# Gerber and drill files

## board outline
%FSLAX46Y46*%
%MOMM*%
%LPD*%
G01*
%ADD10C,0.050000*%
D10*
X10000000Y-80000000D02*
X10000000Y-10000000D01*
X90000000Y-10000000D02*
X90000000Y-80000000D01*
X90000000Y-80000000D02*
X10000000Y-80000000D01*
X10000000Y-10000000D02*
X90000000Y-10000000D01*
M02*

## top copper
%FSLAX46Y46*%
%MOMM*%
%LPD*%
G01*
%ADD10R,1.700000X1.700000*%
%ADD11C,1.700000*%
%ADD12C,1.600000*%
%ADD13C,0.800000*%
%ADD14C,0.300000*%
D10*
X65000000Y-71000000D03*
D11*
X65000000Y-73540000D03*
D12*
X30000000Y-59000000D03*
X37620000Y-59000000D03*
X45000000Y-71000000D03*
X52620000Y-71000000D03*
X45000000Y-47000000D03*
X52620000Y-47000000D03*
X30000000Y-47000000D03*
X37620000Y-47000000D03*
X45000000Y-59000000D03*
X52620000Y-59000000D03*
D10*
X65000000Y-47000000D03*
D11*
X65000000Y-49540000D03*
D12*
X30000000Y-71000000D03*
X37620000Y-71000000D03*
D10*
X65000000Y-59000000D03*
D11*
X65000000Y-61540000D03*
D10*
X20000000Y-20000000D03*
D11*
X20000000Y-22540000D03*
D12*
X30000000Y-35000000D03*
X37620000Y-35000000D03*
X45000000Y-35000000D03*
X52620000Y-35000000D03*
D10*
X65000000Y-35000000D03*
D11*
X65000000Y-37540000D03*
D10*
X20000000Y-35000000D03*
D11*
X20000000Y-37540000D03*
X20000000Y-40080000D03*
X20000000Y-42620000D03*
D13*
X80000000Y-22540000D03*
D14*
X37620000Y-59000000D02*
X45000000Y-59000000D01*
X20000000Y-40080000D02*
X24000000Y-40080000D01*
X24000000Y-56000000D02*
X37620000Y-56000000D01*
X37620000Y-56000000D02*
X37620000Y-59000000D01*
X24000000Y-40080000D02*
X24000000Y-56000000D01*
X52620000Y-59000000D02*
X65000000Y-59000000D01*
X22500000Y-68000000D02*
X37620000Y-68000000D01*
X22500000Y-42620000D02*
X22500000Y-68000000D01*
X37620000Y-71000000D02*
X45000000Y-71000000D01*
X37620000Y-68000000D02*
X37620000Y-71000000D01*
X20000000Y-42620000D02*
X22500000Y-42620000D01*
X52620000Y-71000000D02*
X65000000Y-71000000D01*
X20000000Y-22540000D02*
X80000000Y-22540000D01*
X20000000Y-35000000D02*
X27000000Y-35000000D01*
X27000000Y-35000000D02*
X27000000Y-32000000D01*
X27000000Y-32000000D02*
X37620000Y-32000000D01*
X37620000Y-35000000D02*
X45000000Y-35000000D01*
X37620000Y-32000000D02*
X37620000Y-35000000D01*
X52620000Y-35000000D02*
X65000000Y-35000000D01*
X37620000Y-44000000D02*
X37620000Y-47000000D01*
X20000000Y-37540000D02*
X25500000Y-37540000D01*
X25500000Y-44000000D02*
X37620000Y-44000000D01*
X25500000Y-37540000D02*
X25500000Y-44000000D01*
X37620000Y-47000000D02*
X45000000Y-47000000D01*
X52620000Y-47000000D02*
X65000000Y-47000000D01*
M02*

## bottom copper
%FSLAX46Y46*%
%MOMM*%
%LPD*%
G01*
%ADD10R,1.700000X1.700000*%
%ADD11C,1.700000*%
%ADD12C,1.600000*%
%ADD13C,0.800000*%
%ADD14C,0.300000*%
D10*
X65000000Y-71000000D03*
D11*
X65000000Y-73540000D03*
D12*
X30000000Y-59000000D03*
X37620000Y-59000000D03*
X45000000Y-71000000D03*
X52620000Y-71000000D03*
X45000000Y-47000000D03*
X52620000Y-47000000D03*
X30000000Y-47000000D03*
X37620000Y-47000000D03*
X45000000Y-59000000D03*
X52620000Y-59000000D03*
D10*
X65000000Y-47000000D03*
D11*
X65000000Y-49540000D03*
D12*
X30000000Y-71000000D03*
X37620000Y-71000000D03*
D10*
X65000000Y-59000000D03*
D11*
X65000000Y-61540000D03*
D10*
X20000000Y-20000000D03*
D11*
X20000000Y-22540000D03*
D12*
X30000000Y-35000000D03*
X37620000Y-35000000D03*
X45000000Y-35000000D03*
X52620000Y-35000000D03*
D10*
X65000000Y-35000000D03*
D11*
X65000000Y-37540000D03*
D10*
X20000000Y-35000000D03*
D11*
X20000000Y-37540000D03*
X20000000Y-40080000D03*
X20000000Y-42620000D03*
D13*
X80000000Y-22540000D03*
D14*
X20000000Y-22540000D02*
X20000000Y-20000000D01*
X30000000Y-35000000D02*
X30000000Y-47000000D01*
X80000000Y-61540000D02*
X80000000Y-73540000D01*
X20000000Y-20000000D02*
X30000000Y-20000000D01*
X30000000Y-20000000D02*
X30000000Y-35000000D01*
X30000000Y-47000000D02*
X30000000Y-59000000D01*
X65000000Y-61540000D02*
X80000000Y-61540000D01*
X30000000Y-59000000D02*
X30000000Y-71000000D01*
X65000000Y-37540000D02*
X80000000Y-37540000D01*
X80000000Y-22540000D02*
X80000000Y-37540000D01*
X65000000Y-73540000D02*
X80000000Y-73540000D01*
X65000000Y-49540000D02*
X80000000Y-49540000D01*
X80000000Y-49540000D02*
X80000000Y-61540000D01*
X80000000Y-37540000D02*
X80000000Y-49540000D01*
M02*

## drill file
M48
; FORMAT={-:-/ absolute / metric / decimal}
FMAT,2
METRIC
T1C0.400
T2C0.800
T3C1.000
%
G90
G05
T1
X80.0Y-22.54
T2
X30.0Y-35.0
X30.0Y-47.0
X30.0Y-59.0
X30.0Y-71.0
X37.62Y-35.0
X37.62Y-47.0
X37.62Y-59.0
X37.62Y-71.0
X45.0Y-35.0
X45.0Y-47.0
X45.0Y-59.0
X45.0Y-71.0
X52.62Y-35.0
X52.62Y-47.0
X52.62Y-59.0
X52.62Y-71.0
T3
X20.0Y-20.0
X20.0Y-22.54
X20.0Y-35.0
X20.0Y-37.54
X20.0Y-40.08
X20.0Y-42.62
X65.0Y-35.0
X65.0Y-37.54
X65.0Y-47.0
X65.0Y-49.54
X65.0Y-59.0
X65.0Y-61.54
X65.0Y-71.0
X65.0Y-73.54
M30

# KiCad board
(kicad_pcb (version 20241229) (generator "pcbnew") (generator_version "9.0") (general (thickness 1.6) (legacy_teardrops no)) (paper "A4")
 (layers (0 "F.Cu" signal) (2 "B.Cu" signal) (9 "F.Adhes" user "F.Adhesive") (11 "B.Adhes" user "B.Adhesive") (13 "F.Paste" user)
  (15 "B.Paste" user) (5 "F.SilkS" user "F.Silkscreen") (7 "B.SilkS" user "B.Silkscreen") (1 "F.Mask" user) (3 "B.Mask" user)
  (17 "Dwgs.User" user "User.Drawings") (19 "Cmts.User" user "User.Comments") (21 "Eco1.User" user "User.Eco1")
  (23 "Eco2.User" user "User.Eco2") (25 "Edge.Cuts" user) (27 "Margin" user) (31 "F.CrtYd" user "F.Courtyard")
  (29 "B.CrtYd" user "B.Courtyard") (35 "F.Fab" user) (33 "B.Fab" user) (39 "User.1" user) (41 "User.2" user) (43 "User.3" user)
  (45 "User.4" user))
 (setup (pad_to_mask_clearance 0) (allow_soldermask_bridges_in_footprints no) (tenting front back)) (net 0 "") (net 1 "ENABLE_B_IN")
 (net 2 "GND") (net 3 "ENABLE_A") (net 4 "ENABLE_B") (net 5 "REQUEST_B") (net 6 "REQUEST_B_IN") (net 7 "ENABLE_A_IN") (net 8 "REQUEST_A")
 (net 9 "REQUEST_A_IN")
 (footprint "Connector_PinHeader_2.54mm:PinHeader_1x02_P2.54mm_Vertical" (layer "F.Cu") (at 65 71)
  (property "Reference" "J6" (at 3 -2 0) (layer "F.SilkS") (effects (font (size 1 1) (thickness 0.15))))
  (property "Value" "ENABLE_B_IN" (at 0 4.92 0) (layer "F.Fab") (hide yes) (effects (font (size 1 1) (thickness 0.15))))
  (pad "1" thru_hole rect (at 0 0) (size 1.7 1.7) (drill 1) (layers "*.Cu" "*.Mask") (remove_unused_layers no) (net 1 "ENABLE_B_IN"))
  (pad "2" thru_hole circle (at 0 2.54) (size 1.7 1.7) (drill 1) (layers "*.Cu" "*.Mask") (remove_unused_layers no) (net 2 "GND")))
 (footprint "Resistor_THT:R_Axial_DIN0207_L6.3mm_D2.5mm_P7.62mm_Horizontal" (layer "F.Cu") (at 30 59)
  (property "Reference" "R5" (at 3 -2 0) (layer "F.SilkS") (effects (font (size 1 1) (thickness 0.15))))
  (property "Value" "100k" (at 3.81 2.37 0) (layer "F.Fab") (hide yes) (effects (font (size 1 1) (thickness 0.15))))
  (pad "1" thru_hole circle (at 0 0) (size 1.6 1.6) (drill 0.8) (layers "*.Cu" "*.Mask") (remove_unused_layers no) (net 2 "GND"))
  (pad "2" thru_hole circle (at 7.62 0) (size 1.6 1.6) (drill 0.8) (layers "*.Cu" "*.Mask") (remove_unused_layers no) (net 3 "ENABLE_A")))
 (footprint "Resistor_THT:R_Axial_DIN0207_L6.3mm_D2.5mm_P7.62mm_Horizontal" (layer "F.Cu") (at 45 71)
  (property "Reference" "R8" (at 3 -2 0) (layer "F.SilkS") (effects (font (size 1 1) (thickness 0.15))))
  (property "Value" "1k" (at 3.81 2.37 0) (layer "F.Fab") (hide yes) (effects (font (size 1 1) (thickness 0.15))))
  (pad "1" thru_hole circle (at 0 0) (size 1.6 1.6) (drill 0.8) (layers "*.Cu" "*.Mask") (remove_unused_layers no) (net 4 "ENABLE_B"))
  (pad "2" thru_hole circle (at 7.62 0) (size 1.6 1.6) (drill 0.8) (layers "*.Cu" "*.Mask") (remove_unused_layers no) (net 1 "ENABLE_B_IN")))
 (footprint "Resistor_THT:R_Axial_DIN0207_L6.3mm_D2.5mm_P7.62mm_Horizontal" (layer "F.Cu") (at 45 47)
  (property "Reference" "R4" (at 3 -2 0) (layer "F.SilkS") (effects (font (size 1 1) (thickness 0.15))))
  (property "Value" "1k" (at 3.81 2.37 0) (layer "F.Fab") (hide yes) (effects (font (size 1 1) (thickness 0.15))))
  (pad "1" thru_hole circle (at 0 0) (size 1.6 1.6) (drill 0.8) (layers "*.Cu" "*.Mask") (remove_unused_layers no) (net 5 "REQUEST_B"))
  (pad "2" thru_hole circle (at 7.62 0) (size 1.6 1.6) (drill 0.8) (layers "*.Cu" "*.Mask") (remove_unused_layers no) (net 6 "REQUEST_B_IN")))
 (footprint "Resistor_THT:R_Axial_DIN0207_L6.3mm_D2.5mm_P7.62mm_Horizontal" (layer "F.Cu") (at 30 47)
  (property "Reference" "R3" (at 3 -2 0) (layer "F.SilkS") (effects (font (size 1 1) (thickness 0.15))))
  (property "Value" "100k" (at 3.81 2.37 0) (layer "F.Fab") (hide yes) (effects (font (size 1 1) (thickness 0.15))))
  (pad "1" thru_hole circle (at 0 0) (size 1.6 1.6) (drill 0.8) (layers "*.Cu" "*.Mask") (remove_unused_layers no) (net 2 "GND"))
  (pad "2" thru_hole circle (at 7.62 0) (size 1.6 1.6) (drill 0.8) (layers "*.Cu" "*.Mask") (remove_unused_layers no) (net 5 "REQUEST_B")))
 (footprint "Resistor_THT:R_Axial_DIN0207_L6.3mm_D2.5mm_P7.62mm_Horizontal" (layer "F.Cu") (at 45 59)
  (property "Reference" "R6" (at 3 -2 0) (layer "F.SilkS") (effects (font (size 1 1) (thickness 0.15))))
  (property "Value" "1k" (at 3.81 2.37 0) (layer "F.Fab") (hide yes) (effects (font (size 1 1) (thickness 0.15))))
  (pad "1" thru_hole circle (at 0 0) (size 1.6 1.6) (drill 0.8) (layers "*.Cu" "*.Mask") (remove_unused_layers no) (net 3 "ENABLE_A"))
  (pad "2" thru_hole circle (at 7.62 0) (size 1.6 1.6) (drill 0.8) (layers "*.Cu" "*.Mask") (remove_unused_layers no) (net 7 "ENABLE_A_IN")))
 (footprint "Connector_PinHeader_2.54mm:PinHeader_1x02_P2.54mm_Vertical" (layer "F.Cu") (at 65 47)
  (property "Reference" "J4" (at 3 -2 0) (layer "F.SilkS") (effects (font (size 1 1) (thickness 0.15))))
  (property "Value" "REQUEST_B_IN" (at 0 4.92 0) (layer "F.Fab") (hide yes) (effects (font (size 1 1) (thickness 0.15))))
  (pad "1" thru_hole rect (at 0 0) (size 1.7 1.7) (drill 1) (layers "*.Cu" "*.Mask") (remove_unused_layers no) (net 6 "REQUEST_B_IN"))
  (pad "2" thru_hole circle (at 0 2.54) (size 1.7 1.7) (drill 1) (layers "*.Cu" "*.Mask") (remove_unused_layers no) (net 2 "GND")))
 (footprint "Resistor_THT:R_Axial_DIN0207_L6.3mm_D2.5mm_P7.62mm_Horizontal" (layer "F.Cu") (at 30 71)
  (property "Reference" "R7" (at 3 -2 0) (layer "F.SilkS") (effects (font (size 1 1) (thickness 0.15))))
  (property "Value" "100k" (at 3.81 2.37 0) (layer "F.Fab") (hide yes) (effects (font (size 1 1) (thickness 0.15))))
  (pad "1" thru_hole circle (at 0 0) (size 1.6 1.6) (drill 0.8) (layers "*.Cu" "*.Mask") (remove_unused_layers no) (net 2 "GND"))
  (pad "2" thru_hole circle (at 7.62 0) (size 1.6 1.6) (drill 0.8) (layers "*.Cu" "*.Mask") (remove_unused_layers no) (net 4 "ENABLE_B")))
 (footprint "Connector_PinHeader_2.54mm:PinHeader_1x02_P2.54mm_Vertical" (layer "F.Cu") (at 65 59)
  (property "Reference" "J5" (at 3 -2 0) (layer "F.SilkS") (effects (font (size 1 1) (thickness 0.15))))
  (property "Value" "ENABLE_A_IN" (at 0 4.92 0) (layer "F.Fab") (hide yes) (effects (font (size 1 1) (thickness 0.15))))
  (pad "1" thru_hole rect (at 0 0) (size 1.7 1.7) (drill 1) (layers "*.Cu" "*.Mask") (remove_unused_layers no) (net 7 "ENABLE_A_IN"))
  (pad "2" thru_hole circle (at 0 2.54) (size 1.7 1.7) (drill 1) (layers "*.Cu" "*.Mask") (remove_unused_layers no) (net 2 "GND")))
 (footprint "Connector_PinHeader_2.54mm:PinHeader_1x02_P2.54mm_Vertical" (layer "F.Cu") (at 20 20)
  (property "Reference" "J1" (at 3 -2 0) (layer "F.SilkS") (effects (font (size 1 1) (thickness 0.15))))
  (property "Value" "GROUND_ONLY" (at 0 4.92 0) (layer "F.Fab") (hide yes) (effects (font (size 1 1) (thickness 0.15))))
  (pad "1" thru_hole rect (at 0 0) (size 1.7 1.7) (drill 1) (layers "*.Cu" "*.Mask") (remove_unused_layers no) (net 2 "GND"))
  (pad "2" thru_hole circle (at 0 2.54) (size 1.7 1.7) (drill 1) (layers "*.Cu" "*.Mask") (remove_unused_layers no) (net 2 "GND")))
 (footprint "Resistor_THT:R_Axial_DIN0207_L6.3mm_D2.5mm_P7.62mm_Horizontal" (layer "F.Cu") (at 30 35)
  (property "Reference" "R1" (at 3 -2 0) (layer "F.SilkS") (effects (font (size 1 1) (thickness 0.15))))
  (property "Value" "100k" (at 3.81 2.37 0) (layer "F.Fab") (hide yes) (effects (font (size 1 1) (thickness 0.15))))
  (pad "1" thru_hole circle (at 0 0) (size 1.6 1.6) (drill 0.8) (layers "*.Cu" "*.Mask") (remove_unused_layers no) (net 2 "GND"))
  (pad "2" thru_hole circle (at 7.62 0) (size 1.6 1.6) (drill 0.8) (layers "*.Cu" "*.Mask") (remove_unused_layers no) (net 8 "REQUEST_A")))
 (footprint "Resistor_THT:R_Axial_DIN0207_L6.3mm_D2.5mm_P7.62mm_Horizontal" (layer "F.Cu") (at 45 35)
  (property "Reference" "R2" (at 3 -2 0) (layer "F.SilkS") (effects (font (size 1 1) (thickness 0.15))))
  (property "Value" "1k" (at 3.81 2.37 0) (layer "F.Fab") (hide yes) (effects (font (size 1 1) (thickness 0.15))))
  (pad "1" thru_hole circle (at 0 0) (size 1.6 1.6) (drill 0.8) (layers "*.Cu" "*.Mask") (remove_unused_layers no) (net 8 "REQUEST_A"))
  (pad "2" thru_hole circle (at 7.62 0) (size 1.6 1.6) (drill 0.8) (layers "*.Cu" "*.Mask") (remove_unused_layers no) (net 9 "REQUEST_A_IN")))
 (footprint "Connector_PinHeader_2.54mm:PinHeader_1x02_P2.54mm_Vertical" (layer "F.Cu") (at 65 35)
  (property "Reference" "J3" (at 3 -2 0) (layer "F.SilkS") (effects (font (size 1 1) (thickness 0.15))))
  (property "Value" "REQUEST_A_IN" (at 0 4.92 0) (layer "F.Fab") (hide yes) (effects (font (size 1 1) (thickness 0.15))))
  (pad "1" thru_hole rect (at 0 0) (size 1.7 1.7) (drill 1) (layers "*.Cu" "*.Mask") (remove_unused_layers no) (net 9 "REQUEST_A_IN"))
  (pad "2" thru_hole circle (at 0 2.54) (size 1.7 1.7) (drill 1) (layers "*.Cu" "*.Mask") (remove_unused_layers no) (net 2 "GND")))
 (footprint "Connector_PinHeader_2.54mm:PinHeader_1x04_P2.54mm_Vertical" (layer "F.Cu") (at 20 35)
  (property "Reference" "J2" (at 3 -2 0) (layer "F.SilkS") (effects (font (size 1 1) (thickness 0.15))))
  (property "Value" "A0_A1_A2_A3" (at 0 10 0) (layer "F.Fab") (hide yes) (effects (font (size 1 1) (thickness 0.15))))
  (pad "1" thru_hole rect (at 0 0) (size 1.7 1.7) (drill 1) (layers "*.Cu" "*.Mask") (remove_unused_layers no) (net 8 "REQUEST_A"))
  (pad "2" thru_hole circle (at 0 2.54) (size 1.7 1.7) (drill 1) (layers "*.Cu" "*.Mask") (remove_unused_layers no) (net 5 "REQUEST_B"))
  (pad "3" thru_hole circle (at 0 5.08) (size 1.7 1.7) (drill 1) (layers "*.Cu" "*.Mask") (remove_unused_layers no) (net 3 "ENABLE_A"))
  (pad "4" thru_hole circle (at 0 7.62) (size 1.7 1.7) (drill 1) (layers "*.Cu" "*.Mask") (remove_unused_layers no) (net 4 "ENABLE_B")))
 (gr_line (start 10 80) (end 10 10) (stroke (width 0.05) (type default)) (layer "Edge.Cuts"))
 (gr_line (start 90 10) (end 90 80) (stroke (width 0.05) (type default)) (layer "Edge.Cuts"))
 (gr_line (start 90 80) (end 10 80) (stroke (width 0.05) (type default)) (layer "Edge.Cuts"))
 (gr_line (start 10 10) (end 90 10) (stroke (width 0.05) (type default)) (layer "Edge.Cuts"))
 (segment (start 37.62 59) (end 45 59) (width 0.3) (layer "F.Cu") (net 3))
 (segment (start 20 40.08) (end 24 40.08) (width 0.3) (layer "F.Cu") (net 3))
 (segment (start 24 56) (end 37.62 56) (width 0.3) (layer "F.Cu") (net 3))
 (segment (start 37.62 56) (end 37.62 59) (width 0.3) (layer "F.Cu") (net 3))
 (segment (start 24 40.08) (end 24 56) (width 0.3) (layer "F.Cu") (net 3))
 (segment (start 52.62 59) (end 65 59) (width 0.3) (layer "F.Cu") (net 7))
 (segment (start 22.5 68) (end 37.62 68) (width 0.3) (layer "F.Cu") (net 4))
 (segment (start 22.5 42.62) (end 22.5 68) (width 0.3) (layer "F.Cu") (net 4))
 (segment (start 37.62 71) (end 45 71) (width 0.3) (layer "F.Cu") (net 4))
 (segment (start 37.62 68) (end 37.62 71) (width 0.3) (layer "F.Cu") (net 4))
 (segment (start 20 42.62) (end 22.5 42.62) (width 0.3) (layer "F.Cu") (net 4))
 (segment (start 52.62 71) (end 65 71) (width 0.3) (layer "F.Cu") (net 1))
 (segment (start 20 22.54) (end 80 22.54) (width 0.3) (layer "F.Cu") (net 2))
 (via (at 80 22.54) (size 0.8) (drill 0.4) (layers "F.Cu" "B.Cu") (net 2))
 (segment (start 20 22.54) (end 20 20) (width 0.3) (layer "B.Cu") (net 2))
 (segment (start 30 35) (end 30 47) (width 0.3) (layer "B.Cu") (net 2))
 (segment (start 80 61.54) (end 80 73.54) (width 0.3) (layer "B.Cu") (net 2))
 (segment (start 20 20) (end 30 20) (width 0.3) (layer "B.Cu") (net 2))
 (segment (start 30 20) (end 30 35) (width 0.3) (layer "B.Cu") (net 2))
 (segment (start 30 47) (end 30 59) (width 0.3) (layer "B.Cu") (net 2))
 (segment (start 65 61.54) (end 80 61.54) (width 0.3) (layer "B.Cu") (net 2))
 (segment (start 30 59) (end 30 71) (width 0.3) (layer "B.Cu") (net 2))
 (segment (start 65 37.54) (end 80 37.54) (width 0.3) (layer "B.Cu") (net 2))
 (segment (start 80 22.54) (end 80 37.54) (width 0.3) (layer "B.Cu") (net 2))
 (segment (start 65 73.54) (end 80 73.54) (width 0.3) (layer "B.Cu") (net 2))
 (segment (start 65 49.54) (end 80 49.54) (width 0.3) (layer "B.Cu") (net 2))
 (segment (start 80 49.54) (end 80 61.54) (width 0.3) (layer "B.Cu") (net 2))
 (segment (start 80 37.54) (end 80 49.54) (width 0.3) (layer "B.Cu") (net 2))
 (segment (start 20 35) (end 27 35) (width 0.3) (layer "F.Cu") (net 8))
 (segment (start 27 35) (end 27 32) (width 0.3) (layer "F.Cu") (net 8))
 (segment (start 27 32) (end 37.62 32) (width 0.3) (layer "F.Cu") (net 8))
 (segment (start 37.62 35) (end 45 35) (width 0.3) (layer "F.Cu") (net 8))
 (segment (start 37.62 32) (end 37.62 35) (width 0.3) (layer "F.Cu") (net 8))
 (segment (start 52.62 35) (end 65 35) (width 0.3) (layer "F.Cu") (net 9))
 (segment (start 37.62 44) (end 37.62 47) (width 0.3) (layer "F.Cu") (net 5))
 (segment (start 20 37.54) (end 25.5 37.54) (width 0.3) (layer "F.Cu") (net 5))
 (segment (start 25.5 44) (end 37.62 44) (width 0.3) (layer "F.Cu") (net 5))
 (segment (start 25.5 37.54) (end 25.5 44) (width 0.3) (layer "F.Cu") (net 5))
 (segment (start 37.62 47) (end 45 47) (width 0.3) (layer "F.Cu") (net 5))
 (segment (start 52.62 47) (end 65 47) (width 0.3) (layer "F.Cu") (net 6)))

